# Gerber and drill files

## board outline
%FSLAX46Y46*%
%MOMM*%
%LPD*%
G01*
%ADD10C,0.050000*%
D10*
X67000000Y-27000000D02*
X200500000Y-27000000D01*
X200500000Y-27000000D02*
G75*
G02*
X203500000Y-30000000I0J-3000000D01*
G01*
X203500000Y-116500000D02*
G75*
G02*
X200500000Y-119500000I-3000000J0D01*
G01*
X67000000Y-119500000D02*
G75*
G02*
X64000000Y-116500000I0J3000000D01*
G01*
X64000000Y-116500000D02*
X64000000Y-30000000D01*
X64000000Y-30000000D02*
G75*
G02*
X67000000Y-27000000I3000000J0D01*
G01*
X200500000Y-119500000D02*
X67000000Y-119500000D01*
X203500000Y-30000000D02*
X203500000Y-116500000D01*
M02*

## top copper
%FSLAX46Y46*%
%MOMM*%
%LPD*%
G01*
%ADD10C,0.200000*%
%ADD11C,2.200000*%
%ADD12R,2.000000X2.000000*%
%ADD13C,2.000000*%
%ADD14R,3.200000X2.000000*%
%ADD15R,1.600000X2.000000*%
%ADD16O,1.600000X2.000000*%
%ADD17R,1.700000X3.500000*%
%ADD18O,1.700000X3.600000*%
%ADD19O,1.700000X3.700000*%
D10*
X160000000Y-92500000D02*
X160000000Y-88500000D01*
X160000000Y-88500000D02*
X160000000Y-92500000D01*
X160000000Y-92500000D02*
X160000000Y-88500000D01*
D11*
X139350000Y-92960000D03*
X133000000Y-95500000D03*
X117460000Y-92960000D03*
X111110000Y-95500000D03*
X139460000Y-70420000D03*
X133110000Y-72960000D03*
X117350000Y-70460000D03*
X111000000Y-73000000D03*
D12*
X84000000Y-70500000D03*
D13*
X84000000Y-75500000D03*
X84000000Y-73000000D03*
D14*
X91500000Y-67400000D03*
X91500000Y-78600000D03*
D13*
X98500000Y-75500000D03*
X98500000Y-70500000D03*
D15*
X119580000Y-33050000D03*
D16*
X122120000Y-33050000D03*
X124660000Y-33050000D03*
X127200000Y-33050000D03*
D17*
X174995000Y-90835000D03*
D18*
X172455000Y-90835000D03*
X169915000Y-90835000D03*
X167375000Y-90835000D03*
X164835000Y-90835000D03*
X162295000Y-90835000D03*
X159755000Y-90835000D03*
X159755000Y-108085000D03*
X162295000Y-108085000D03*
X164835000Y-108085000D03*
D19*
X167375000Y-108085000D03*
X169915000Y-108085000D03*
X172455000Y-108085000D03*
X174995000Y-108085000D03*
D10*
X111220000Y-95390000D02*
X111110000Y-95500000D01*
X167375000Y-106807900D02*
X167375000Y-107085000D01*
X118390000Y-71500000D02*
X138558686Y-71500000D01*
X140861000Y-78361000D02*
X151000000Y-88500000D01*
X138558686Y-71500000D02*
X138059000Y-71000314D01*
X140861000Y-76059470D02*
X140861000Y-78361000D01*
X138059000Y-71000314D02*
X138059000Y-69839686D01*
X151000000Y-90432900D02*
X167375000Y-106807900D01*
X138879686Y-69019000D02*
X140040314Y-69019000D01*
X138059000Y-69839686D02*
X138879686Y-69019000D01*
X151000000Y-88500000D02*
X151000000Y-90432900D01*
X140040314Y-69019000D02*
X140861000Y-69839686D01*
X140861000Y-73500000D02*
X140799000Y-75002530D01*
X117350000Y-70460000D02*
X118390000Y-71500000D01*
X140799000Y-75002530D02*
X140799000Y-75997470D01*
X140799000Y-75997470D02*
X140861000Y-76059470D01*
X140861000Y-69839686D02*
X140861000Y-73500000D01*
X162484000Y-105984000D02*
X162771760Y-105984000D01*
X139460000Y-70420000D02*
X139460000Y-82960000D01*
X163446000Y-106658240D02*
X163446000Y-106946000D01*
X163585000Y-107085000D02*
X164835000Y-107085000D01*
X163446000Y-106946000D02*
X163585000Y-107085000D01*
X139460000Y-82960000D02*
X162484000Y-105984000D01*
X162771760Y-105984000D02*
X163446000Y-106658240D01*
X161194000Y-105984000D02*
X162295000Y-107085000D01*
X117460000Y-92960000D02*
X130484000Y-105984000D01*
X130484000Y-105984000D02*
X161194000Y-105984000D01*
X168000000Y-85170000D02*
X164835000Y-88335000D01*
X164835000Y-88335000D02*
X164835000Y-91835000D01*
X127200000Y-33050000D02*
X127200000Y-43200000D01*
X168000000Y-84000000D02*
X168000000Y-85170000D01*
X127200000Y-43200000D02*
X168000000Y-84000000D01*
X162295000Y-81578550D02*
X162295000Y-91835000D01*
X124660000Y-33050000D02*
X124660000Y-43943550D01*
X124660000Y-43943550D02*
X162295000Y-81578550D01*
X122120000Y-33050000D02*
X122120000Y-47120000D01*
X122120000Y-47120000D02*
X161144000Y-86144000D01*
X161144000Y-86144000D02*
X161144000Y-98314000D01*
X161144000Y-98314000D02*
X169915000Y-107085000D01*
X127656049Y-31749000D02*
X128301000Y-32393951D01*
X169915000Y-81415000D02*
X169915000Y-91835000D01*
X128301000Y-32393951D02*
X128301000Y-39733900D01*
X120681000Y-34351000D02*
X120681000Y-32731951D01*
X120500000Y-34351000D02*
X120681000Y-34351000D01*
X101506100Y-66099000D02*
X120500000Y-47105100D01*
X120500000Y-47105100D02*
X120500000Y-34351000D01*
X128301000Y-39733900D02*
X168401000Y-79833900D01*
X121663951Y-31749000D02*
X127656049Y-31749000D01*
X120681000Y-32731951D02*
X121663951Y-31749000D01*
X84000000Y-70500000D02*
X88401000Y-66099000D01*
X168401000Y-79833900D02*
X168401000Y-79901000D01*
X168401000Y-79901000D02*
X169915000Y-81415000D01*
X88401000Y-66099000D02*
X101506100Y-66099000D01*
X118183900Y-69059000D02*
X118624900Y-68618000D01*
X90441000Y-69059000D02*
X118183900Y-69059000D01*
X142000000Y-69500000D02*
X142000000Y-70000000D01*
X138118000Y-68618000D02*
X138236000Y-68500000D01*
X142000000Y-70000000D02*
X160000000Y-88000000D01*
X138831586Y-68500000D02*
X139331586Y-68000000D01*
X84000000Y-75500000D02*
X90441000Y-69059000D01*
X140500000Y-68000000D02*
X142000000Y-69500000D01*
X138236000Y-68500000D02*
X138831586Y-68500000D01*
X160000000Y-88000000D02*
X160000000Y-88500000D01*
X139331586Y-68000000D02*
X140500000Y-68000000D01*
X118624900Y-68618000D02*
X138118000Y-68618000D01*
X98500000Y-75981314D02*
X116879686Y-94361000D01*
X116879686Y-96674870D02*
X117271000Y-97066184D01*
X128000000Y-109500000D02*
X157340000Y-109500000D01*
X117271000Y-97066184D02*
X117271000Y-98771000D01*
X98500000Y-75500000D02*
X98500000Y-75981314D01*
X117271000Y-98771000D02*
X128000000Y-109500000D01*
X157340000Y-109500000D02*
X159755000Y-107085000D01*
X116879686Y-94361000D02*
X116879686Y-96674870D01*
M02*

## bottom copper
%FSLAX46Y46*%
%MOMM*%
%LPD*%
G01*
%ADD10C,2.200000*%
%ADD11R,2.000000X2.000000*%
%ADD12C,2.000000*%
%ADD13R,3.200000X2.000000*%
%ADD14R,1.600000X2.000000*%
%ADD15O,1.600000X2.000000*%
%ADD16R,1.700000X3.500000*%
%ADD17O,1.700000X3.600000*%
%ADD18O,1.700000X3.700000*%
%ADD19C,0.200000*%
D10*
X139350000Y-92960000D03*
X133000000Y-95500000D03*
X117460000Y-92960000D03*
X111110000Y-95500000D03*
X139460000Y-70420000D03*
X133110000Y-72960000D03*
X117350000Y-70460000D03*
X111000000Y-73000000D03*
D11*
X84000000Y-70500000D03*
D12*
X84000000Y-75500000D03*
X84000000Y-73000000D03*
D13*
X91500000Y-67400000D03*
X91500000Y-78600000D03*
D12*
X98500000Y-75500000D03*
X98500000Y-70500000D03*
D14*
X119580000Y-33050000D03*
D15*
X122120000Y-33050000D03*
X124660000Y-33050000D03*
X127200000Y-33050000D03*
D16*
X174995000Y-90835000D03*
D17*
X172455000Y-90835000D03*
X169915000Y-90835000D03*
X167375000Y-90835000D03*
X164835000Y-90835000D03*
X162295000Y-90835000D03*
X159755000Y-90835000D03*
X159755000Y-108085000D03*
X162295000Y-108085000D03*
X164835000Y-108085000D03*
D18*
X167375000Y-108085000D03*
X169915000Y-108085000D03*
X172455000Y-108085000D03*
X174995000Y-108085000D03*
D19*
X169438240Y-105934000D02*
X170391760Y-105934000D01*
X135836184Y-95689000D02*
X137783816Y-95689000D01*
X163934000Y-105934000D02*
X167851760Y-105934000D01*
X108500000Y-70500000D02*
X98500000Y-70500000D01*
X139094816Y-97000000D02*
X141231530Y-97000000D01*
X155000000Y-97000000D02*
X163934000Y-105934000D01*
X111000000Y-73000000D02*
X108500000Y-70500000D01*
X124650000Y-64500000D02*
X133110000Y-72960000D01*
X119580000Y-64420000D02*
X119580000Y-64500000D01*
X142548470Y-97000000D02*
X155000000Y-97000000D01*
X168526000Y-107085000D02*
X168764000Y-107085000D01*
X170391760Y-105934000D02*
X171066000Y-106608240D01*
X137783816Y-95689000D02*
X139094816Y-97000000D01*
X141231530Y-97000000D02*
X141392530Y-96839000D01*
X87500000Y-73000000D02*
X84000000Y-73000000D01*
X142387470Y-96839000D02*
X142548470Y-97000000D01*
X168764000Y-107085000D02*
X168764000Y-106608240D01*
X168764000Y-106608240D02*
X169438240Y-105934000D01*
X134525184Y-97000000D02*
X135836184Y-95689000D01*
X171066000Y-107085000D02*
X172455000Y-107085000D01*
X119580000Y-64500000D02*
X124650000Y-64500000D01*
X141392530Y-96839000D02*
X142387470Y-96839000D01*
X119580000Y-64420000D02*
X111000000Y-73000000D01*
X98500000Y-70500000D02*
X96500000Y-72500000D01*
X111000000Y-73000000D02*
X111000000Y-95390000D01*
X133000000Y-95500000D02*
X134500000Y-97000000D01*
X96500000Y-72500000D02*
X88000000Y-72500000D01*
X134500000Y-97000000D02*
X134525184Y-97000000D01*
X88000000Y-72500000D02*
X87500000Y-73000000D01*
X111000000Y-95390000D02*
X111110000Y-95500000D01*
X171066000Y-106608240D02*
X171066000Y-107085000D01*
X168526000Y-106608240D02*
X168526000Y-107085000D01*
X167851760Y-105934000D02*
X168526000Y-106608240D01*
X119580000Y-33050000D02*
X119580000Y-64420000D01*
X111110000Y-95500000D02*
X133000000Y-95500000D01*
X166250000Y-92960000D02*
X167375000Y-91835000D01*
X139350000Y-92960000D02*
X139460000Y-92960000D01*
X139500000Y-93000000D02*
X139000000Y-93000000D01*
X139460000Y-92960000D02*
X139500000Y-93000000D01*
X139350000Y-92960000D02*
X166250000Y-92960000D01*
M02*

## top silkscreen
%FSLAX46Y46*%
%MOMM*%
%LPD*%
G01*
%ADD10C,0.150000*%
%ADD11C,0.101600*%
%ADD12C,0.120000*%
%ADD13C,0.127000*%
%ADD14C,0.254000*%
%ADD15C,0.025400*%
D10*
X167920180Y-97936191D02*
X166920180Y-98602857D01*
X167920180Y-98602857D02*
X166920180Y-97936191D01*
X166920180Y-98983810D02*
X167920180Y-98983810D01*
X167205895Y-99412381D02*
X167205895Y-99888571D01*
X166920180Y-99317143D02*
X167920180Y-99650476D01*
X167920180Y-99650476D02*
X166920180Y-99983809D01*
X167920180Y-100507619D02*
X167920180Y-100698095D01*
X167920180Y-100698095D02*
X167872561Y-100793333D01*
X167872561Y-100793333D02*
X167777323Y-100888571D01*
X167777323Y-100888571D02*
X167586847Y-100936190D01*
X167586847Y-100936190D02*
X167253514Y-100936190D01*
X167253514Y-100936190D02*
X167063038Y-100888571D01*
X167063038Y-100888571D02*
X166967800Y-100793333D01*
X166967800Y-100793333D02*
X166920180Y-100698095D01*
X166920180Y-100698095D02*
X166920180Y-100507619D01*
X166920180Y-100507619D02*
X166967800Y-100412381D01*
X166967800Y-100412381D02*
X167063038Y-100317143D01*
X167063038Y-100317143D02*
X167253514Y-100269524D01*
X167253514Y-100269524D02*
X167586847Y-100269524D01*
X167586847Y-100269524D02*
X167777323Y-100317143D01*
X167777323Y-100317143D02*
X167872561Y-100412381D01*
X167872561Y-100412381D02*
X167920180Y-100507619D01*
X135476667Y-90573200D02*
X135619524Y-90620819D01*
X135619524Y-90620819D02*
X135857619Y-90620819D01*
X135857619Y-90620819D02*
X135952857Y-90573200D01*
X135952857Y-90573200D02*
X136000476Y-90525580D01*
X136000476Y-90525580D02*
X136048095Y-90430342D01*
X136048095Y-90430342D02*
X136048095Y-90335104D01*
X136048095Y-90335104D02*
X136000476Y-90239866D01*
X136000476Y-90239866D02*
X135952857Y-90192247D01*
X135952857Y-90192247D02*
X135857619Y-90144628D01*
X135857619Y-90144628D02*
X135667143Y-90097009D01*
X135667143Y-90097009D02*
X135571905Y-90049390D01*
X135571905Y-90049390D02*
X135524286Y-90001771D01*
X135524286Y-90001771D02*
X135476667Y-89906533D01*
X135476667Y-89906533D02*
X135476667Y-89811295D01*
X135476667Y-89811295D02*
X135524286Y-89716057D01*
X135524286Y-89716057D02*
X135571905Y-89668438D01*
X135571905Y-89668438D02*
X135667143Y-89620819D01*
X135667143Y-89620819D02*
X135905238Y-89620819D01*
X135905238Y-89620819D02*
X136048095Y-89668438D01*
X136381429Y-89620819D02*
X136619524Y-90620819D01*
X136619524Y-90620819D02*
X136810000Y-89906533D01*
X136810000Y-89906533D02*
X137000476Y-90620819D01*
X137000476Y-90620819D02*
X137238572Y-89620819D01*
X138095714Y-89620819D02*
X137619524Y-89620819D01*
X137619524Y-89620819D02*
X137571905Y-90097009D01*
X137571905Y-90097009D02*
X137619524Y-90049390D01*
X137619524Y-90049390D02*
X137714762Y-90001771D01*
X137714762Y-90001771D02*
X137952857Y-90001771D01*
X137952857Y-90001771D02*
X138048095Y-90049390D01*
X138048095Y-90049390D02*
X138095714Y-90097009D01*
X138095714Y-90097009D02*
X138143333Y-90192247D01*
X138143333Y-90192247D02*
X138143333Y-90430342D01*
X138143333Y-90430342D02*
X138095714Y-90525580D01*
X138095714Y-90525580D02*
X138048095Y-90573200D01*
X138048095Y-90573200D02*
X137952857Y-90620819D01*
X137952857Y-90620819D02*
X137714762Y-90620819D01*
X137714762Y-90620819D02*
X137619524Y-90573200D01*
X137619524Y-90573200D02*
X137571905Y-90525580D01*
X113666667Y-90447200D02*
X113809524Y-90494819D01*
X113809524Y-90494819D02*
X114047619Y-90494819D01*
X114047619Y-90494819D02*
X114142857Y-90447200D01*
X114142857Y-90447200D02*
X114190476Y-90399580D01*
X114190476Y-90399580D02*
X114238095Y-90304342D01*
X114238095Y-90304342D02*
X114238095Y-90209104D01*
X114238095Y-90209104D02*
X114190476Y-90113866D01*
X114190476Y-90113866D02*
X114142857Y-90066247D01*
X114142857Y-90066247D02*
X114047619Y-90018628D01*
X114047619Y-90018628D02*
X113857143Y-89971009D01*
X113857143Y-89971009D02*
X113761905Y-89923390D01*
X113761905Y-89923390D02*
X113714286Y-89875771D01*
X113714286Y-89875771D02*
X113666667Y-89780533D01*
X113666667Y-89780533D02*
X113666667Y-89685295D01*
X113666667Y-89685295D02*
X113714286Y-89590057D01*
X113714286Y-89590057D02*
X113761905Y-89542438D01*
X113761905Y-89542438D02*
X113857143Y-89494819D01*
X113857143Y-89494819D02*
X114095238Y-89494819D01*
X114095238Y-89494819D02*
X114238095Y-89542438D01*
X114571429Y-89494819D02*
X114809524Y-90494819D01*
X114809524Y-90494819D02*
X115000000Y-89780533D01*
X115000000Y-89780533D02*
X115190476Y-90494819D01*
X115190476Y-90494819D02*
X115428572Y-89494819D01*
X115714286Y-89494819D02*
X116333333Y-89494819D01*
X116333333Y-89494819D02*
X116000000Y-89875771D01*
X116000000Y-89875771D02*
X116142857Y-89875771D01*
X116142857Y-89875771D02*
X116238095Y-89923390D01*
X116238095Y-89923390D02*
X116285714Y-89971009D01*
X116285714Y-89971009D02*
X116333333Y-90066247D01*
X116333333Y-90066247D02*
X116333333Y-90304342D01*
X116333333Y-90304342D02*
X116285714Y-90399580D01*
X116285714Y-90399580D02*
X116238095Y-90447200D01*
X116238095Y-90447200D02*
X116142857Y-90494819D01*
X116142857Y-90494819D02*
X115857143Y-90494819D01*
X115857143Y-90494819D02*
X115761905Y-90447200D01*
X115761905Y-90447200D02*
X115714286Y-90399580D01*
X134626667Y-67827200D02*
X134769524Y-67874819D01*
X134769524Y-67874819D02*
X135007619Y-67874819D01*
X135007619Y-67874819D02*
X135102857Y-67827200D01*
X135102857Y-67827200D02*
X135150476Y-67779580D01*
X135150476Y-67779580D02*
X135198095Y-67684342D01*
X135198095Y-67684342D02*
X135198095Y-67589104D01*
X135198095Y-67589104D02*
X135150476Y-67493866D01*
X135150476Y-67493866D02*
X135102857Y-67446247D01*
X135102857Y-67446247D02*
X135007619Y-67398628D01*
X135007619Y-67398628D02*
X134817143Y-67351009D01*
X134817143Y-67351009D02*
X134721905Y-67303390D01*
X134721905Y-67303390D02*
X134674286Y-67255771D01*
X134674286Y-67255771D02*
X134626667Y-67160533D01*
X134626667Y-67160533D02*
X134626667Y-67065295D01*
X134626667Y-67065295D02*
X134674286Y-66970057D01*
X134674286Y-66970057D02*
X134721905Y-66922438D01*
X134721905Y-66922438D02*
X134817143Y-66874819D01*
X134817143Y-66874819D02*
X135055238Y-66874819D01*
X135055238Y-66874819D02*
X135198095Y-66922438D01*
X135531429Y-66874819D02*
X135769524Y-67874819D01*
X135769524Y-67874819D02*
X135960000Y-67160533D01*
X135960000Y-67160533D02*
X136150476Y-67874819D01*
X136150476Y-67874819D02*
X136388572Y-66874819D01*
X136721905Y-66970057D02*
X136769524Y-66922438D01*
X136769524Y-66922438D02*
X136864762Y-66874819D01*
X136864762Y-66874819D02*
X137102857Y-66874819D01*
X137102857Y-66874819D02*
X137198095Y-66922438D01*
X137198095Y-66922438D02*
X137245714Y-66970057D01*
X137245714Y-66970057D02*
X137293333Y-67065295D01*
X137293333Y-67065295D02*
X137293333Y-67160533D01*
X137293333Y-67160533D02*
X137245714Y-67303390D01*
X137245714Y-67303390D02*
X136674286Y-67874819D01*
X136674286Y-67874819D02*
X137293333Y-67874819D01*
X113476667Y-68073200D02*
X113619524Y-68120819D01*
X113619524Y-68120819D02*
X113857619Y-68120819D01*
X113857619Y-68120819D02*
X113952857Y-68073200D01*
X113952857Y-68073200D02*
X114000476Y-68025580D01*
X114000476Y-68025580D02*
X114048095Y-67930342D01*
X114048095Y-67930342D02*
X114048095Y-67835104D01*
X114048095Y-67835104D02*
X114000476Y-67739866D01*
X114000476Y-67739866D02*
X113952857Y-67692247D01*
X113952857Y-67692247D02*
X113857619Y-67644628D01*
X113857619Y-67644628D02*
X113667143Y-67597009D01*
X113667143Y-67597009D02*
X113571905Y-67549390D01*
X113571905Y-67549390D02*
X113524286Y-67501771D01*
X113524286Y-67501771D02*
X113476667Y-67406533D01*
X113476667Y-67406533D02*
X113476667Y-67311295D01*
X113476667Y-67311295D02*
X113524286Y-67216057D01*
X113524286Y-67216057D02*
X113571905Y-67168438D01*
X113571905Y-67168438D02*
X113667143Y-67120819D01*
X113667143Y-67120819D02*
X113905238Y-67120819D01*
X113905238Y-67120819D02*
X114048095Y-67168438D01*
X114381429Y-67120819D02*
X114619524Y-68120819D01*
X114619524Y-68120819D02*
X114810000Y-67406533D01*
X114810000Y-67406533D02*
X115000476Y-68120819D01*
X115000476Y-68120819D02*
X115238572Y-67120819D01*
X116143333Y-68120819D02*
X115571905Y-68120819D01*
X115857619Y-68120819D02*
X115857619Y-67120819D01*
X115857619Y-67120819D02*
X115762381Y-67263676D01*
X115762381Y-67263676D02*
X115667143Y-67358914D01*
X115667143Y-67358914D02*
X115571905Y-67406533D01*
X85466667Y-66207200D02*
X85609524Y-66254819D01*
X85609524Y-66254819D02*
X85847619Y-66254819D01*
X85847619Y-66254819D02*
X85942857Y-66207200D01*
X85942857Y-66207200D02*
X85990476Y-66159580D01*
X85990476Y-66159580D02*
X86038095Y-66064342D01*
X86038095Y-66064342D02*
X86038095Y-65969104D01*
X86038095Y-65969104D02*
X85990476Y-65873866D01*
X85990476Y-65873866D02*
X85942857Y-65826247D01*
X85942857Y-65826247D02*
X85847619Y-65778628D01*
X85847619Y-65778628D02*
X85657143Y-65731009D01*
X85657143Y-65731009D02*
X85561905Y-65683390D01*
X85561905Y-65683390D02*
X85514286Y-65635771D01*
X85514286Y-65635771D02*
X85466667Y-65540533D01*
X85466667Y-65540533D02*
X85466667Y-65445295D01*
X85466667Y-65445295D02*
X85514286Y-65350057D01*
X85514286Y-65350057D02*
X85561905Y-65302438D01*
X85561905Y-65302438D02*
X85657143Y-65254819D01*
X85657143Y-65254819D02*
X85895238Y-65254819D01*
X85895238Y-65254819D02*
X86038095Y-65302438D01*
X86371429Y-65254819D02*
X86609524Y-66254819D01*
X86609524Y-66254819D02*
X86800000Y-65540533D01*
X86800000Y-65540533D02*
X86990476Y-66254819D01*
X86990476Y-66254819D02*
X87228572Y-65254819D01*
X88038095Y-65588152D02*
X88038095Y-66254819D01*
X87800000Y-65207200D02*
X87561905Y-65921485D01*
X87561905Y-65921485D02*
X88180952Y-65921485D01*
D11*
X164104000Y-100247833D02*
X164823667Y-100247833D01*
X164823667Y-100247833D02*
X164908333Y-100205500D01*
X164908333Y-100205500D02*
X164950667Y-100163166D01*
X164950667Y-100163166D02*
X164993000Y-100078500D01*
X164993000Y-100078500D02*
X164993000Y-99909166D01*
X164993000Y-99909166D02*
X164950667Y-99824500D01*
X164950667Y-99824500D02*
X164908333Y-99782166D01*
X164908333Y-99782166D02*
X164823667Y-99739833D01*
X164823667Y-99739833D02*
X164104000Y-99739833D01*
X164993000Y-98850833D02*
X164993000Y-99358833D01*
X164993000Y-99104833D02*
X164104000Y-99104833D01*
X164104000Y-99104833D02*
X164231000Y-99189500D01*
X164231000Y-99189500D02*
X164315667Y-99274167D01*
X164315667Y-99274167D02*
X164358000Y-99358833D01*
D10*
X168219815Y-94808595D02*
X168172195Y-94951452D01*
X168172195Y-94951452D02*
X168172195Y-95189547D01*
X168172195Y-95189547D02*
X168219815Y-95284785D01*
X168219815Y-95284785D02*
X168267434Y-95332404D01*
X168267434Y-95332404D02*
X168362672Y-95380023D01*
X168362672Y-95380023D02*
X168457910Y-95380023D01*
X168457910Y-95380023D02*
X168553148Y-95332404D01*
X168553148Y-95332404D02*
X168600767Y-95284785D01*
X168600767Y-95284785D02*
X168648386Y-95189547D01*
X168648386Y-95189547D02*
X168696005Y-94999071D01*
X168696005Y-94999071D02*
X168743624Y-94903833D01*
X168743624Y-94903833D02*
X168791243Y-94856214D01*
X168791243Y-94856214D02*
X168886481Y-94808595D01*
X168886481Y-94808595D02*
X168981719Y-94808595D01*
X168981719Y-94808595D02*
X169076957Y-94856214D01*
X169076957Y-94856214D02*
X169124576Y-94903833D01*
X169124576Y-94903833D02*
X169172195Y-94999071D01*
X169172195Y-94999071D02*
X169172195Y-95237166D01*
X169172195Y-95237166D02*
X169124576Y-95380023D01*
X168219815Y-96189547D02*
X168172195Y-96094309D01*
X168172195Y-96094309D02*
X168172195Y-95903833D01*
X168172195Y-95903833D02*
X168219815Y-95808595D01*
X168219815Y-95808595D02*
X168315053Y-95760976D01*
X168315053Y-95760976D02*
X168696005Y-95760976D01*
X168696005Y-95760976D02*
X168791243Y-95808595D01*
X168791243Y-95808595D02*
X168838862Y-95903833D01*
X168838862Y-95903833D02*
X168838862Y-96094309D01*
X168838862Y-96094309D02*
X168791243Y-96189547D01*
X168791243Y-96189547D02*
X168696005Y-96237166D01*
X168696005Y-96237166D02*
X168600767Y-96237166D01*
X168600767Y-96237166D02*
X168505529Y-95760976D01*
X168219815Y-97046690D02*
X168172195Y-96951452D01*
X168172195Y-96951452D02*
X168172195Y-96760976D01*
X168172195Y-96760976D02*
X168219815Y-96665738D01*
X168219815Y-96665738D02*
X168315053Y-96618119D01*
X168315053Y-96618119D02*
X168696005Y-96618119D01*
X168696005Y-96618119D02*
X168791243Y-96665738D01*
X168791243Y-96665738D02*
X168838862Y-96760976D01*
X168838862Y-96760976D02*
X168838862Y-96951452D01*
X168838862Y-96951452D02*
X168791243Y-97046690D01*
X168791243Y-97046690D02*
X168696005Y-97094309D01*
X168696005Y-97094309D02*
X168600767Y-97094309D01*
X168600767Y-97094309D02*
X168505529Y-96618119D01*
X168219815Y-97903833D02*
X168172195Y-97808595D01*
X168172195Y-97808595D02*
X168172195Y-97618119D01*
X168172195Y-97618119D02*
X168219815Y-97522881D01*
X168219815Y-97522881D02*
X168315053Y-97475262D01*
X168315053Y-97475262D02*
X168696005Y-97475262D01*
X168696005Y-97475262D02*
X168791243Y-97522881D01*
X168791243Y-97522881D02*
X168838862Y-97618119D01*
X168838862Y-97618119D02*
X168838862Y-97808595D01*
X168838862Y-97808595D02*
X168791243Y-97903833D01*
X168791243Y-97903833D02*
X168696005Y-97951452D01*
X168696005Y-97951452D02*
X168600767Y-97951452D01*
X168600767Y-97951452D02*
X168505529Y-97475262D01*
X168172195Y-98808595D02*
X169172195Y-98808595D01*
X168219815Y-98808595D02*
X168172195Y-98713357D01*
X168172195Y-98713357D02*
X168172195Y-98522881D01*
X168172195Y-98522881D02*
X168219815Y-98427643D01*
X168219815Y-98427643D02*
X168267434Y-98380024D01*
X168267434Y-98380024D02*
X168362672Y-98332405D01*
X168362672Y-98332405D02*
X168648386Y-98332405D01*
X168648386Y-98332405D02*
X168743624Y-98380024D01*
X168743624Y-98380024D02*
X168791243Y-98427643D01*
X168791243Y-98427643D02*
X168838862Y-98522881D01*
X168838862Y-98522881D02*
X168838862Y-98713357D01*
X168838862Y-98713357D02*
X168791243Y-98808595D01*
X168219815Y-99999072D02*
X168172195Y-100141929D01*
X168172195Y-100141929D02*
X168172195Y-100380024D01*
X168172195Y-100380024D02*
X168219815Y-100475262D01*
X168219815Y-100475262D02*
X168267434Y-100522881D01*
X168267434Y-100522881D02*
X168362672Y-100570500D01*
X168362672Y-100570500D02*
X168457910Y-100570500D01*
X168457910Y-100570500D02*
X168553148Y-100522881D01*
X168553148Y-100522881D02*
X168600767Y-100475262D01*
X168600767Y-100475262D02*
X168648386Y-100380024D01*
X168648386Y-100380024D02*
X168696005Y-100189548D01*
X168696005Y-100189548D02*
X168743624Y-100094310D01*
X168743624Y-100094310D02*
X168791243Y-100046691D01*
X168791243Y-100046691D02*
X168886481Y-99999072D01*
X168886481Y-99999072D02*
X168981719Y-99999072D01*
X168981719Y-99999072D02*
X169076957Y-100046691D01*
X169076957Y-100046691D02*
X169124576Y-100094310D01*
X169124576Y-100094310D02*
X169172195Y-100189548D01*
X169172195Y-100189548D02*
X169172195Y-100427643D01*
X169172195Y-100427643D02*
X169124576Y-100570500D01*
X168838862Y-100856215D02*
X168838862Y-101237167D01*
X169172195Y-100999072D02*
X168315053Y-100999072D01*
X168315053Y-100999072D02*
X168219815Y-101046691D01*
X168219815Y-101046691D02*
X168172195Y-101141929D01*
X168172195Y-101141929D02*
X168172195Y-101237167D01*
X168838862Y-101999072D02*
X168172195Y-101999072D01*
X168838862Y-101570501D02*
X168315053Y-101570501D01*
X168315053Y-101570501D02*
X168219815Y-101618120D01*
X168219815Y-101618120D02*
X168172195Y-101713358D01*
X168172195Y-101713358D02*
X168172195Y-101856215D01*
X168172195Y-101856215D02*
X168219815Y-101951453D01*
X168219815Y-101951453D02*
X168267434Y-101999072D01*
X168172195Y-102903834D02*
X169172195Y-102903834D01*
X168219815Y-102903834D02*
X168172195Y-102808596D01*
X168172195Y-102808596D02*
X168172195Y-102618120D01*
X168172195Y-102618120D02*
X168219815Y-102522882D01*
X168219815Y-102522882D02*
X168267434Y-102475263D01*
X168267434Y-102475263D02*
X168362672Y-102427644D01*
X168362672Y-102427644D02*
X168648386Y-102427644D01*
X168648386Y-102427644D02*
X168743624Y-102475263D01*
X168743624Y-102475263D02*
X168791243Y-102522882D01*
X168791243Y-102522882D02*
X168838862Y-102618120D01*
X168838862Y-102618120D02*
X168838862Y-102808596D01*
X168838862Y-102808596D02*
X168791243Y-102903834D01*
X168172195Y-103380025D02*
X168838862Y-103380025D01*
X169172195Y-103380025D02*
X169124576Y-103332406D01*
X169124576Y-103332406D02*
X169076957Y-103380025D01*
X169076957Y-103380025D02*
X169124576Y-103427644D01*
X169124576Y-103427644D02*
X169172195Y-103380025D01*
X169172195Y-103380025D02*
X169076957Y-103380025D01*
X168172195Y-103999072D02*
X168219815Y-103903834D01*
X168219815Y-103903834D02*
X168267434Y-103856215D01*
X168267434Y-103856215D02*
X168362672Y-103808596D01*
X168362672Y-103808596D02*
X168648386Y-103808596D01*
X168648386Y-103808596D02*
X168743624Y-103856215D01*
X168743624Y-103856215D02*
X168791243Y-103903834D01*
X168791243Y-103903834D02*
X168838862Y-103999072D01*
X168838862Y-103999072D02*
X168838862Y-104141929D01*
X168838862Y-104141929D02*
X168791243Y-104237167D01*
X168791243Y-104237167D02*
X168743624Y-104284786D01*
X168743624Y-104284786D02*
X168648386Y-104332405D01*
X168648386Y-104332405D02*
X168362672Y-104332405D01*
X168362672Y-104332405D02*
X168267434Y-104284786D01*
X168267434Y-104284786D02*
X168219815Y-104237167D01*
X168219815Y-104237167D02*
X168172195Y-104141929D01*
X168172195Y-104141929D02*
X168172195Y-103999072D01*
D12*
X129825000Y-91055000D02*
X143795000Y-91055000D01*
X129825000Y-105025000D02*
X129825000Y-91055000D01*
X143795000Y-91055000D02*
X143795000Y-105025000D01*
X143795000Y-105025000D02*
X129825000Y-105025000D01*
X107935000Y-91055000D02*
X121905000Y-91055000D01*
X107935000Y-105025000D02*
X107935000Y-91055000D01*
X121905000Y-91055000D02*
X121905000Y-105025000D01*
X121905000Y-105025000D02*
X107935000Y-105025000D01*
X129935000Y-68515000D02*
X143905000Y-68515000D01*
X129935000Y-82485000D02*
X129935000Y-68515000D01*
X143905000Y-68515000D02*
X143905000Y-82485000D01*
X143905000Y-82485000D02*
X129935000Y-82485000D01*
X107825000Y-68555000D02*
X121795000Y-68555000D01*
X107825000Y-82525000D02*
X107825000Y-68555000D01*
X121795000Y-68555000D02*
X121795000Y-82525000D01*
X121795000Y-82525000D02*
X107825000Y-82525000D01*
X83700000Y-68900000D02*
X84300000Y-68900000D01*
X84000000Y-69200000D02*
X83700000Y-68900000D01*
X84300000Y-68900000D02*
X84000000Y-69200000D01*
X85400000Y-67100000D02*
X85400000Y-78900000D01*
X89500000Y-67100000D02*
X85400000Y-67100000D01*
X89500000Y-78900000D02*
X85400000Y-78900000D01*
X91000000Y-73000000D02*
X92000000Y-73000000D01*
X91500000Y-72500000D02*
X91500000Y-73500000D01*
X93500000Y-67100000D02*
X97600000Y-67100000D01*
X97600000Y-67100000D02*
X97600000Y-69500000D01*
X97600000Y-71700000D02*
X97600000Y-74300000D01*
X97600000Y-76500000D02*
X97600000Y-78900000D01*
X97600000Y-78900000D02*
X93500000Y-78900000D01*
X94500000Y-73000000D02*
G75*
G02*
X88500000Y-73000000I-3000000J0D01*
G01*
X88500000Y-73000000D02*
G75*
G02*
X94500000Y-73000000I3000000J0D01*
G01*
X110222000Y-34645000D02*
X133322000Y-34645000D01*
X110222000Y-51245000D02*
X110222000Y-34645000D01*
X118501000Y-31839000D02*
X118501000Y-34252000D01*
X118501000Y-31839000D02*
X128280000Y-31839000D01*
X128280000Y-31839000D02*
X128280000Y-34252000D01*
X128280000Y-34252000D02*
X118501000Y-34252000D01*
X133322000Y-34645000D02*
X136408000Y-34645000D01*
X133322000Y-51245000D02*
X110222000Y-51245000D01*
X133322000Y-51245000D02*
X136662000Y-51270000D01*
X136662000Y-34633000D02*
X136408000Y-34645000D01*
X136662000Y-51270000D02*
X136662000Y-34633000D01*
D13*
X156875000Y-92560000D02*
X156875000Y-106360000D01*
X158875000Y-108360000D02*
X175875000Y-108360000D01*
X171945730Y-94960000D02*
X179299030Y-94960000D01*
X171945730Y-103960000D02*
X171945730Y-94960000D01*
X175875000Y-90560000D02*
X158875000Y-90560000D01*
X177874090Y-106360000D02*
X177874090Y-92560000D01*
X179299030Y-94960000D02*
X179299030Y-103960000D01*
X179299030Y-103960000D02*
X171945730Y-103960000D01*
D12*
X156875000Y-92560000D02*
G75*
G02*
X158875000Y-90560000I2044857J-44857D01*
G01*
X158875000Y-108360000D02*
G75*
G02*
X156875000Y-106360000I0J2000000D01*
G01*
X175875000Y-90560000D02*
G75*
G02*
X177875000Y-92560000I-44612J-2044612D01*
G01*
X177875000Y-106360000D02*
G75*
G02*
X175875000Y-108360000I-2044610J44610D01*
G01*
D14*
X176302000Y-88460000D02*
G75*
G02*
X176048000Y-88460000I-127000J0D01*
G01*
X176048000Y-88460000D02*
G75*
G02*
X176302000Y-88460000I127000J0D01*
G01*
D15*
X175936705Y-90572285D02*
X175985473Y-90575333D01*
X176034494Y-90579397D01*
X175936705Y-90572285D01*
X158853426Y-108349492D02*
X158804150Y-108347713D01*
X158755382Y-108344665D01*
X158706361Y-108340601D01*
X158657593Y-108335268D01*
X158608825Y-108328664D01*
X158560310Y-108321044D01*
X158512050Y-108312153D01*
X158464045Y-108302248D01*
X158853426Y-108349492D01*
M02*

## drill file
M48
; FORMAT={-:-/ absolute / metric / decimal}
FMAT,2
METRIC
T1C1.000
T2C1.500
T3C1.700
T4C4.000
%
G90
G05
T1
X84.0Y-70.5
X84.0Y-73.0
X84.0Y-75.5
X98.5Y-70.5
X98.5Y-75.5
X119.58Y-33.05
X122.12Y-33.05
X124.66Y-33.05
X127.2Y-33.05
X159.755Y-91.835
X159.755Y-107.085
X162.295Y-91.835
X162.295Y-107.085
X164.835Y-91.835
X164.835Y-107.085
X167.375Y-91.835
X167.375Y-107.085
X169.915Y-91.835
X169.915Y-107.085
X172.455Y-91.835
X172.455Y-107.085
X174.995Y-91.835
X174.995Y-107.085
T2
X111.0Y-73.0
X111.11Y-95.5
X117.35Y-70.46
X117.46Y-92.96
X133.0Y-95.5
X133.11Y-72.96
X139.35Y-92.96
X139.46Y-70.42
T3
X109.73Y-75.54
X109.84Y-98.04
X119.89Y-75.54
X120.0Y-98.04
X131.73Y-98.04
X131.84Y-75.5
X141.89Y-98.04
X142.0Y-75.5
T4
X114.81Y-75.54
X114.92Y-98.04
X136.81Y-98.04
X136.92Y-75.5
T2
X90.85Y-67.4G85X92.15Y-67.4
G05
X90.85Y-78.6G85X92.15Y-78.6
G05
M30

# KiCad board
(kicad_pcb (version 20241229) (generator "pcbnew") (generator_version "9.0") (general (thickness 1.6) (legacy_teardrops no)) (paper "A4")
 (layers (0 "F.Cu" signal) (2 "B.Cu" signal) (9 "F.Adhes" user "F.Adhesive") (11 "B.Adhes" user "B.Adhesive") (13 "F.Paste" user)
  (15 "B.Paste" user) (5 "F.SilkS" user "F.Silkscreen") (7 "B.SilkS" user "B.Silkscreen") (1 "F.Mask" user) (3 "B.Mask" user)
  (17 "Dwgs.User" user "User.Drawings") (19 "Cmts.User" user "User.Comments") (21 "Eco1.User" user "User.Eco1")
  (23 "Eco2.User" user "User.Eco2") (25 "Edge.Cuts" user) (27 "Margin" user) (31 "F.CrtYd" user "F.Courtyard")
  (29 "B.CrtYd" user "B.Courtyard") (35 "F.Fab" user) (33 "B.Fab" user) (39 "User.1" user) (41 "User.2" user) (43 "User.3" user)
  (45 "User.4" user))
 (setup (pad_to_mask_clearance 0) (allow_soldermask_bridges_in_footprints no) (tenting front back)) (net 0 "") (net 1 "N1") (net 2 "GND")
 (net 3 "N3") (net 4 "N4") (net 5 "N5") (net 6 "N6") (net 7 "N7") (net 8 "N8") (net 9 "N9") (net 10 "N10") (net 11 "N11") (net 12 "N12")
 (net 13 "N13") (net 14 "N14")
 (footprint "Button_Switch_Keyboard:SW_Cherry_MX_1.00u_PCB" (layer "F.Cu") (at 139.35 92.96)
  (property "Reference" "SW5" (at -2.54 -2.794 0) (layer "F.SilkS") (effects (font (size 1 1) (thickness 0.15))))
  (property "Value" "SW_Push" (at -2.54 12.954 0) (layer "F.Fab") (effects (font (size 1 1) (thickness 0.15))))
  (fp_line (start -9.525 -1.905) (end 4.445 -1.905) (stroke (width 0.12) (type solid)) (layer "F.SilkS"))
  (fp_line (start -9.525 12.065) (end -9.525 -1.905) (stroke (width 0.12) (type solid)) (layer "F.SilkS"))
  (fp_line (start 4.445 -1.905) (end 4.445 12.065) (stroke (width 0.12) (type solid)) (layer "F.SilkS"))
  (fp_line (start 4.445 12.065) (end -9.525 12.065) (stroke (width 0.12) (type solid)) (layer "F.SilkS"))
  (pad "" np_thru_hole circle (at -7.62 5.08) (size 1.7 1.7) (drill 1.7) (layers "*.Cu" "*.Mask"))
  (pad "" np_thru_hole circle (at -2.54 5.08) (size 4 4) (drill 4) (layers "*.Cu" "*.Mask"))
  (pad "" np_thru_hole circle (at 2.54 5.08) (size 1.7 1.7) (drill 1.7) (layers "*.Cu" "*.Mask"))
  (pad "1" thru_hole circle (at 0 0) (size 2.2 2.2) (drill 1.5) (layers "*.Cu" "*.Mask") (remove_unused_layers no) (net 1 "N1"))
  (pad "2" thru_hole circle (at -6.35 2.54) (size 2.2 2.2) (drill 1.5) (layers "*.Cu" "*.Mask") (remove_unused_layers no) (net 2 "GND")))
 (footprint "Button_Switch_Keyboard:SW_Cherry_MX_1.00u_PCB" (layer "F.Cu") (at 117.46 92.96)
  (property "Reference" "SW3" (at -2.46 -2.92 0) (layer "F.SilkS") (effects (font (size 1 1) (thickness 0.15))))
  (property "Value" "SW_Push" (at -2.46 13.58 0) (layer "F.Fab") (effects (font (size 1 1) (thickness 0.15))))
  (fp_line (start -9.525 -1.905) (end 4.445 -1.905) (stroke (width 0.12) (type solid)) (layer "F.SilkS"))
  (fp_line (start -9.525 12.065) (end -9.525 -1.905) (stroke (width 0.12) (type solid)) (layer "F.SilkS"))
  (fp_line (start 4.445 -1.905) (end 4.445 12.065) (stroke (width 0.12) (type solid)) (layer "F.SilkS"))
  (fp_line (start 4.445 12.065) (end -9.525 12.065) (stroke (width 0.12) (type solid)) (layer "F.SilkS"))
  (pad "" np_thru_hole circle (at -7.62 5.08) (size 1.7 1.7) (drill 1.7) (layers "*.Cu" "*.Mask"))
  (pad "" np_thru_hole circle (at -2.54 5.08) (size 4 4) (drill 4) (layers "*.Cu" "*.Mask"))
  (pad "" np_thru_hole circle (at 2.54 5.08) (size 1.7 1.7) (drill 1.7) (layers "*.Cu" "*.Mask"))
  (pad "1" thru_hole circle (at 0 0) (size 2.2 2.2) (drill 1.5) (layers "*.Cu" "*.Mask") (remove_unused_layers no) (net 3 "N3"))
  (pad "2" thru_hole circle (at -6.35 2.54) (size 2.2 2.2) (drill 1.5) (layers "*.Cu" "*.Mask") (remove_unused_layers no) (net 2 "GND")))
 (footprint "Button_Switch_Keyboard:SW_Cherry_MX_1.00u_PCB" (layer "F.Cu") (at 139.46 70.42)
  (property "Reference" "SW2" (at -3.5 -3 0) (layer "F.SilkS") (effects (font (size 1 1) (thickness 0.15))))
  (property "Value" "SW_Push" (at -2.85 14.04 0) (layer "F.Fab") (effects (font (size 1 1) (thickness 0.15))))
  (fp_line (start -9.525 -1.905) (end 4.445 -1.905) (stroke (width 0.12) (type solid)) (layer "F.SilkS"))
  (fp_line (start -9.525 12.065) (end -9.525 -1.905) (stroke (width 0.12) (type solid)) (layer "F.SilkS"))
  (fp_line (start 4.445 -1.905) (end 4.445 12.065) (stroke (width 0.12) (type solid)) (layer "F.SilkS"))
  (fp_line (start 4.445 12.065) (end -9.525 12.065) (stroke (width 0.12) (type solid)) (layer "F.SilkS"))
  (pad "" np_thru_hole circle (at -7.62 5.08) (size 1.7 1.7) (drill 1.7) (layers "*.Cu" "*.Mask"))
  (pad "" np_thru_hole circle (at -2.54 5.08) (size 4 4) (drill 4) (layers "*.Cu" "*.Mask"))
  (pad "" np_thru_hole circle (at 2.54 5.08) (size 1.7 1.7) (drill 1.7) (layers "*.Cu" "*.Mask"))
  (pad "1" thru_hole circle (at 0 0) (size 2.2 2.2) (drill 1.5) (layers "*.Cu" "*.Mask") (remove_unused_layers no) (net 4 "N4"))
  (pad "2" thru_hole circle (at -6.35 2.54) (size 2.2 2.2) (drill 1.5) (layers "*.Cu" "*.Mask") (remove_unused_layers no) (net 2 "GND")))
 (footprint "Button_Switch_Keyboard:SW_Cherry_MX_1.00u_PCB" (layer "F.Cu") (at 117.35 70.46)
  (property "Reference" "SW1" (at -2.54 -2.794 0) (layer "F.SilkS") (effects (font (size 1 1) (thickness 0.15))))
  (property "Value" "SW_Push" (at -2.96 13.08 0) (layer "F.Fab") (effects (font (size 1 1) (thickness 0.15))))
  (fp_line (start -9.525 -1.905) (end 4.445 -1.905) (stroke (width 0.12) (type solid)) (layer "F.SilkS"))
  (fp_line (start -9.525 12.065) (end -9.525 -1.905) (stroke (width 0.12) (type solid)) (layer "F.SilkS"))
  (fp_line (start 4.445 -1.905) (end 4.445 12.065) (stroke (width 0.12) (type solid)) (layer "F.SilkS"))
  (fp_line (start 4.445 12.065) (end -9.525 12.065) (stroke (width 0.12) (type solid)) (layer "F.SilkS"))
  (pad "" np_thru_hole circle (at -7.62 5.08) (size 1.7 1.7) (drill 1.7) (layers "*.Cu" "*.Mask"))
  (pad "" np_thru_hole circle (at -2.54 5.08) (size 4 4) (drill 4) (layers "*.Cu" "*.Mask"))
  (pad "" np_thru_hole circle (at 2.54 5.08) (size 1.7 1.7) (drill 1.7) (layers "*.Cu" "*.Mask"))
  (pad "1" thru_hole circle (at 0 0) (size 2.2 2.2) (drill 1.5) (layers "*.Cu" "*.Mask") (remove_unused_layers no) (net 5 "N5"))
  (pad "2" thru_hole circle (at -6.35 2.54) (size 2.2 2.2) (drill 1.5) (layers "*.Cu" "*.Mask") (remove_unused_layers no) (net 2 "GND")))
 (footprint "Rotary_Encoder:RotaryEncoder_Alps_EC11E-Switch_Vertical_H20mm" (layer "F.Cu") (at 84 70.5)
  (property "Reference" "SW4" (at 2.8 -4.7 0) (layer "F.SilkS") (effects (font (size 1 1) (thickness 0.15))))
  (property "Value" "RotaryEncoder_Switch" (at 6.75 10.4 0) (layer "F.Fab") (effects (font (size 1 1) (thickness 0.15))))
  (fp_line (start -0.3 -1.6) (end 0.3 -1.6) (stroke (width 0.12) (type solid)) (layer "F.SilkS"))
  (fp_line (start 0 -1.3) (end -0.3 -1.6) (stroke (width 0.12) (type solid)) (layer "F.SilkS"))
  (fp_line (start 0.3 -1.6) (end 0 -1.3) (stroke (width 0.12) (type solid)) (layer "F.SilkS"))
  (fp_line (start 1.4 -3.4) (end 1.4 8.4) (stroke (width 0.12) (type solid)) (layer "F.SilkS"))
  (fp_line (start 5.5 -3.4) (end 1.4 -3.4) (stroke (width 0.12) (type solid)) (layer "F.SilkS"))
  (fp_line (start 5.5 8.4) (end 1.4 8.4) (stroke (width 0.12) (type solid)) (layer "F.SilkS"))
  (fp_line (start 7 2.5) (end 8 2.5) (stroke (width 0.12) (type solid)) (layer "F.SilkS"))
  (fp_line (start 7.5 2) (end 7.5 3) (stroke (width 0.12) (type solid)) (layer "F.SilkS"))
  (fp_line (start 9.5 -3.4) (end 13.6 -3.4) (stroke (width 0.12) (type solid)) (layer "F.SilkS"))
  (fp_line (start 13.6 -3.4) (end 13.6 -1) (stroke (width 0.12) (type solid)) (layer "F.SilkS"))
  (fp_line (start 13.6 1.2) (end 13.6 3.8) (stroke (width 0.12) (type solid)) (layer "F.SilkS"))
  (fp_line (start 13.6 6) (end 13.6 8.4) (stroke (width 0.12) (type solid)) (layer "F.SilkS"))
  (fp_line (start 13.6 8.4) (end 9.5 8.4) (stroke (width 0.12) (type solid)) (layer "F.SilkS"))
  (fp_circle (center 7.5 2.5) (end 10.5 2.5) (stroke (width 0.12) (type solid)) (fill no) (layer "F.SilkS"))
  (pad "A" thru_hole rect (at 0 0) (size 2 2) (drill 1) (layers "*.Cu" "*.Mask") (remove_unused_layers no) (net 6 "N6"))
  (pad "B" thru_hole circle (at 0 5) (size 2 2) (drill 1) (layers "*.Cu" "*.Mask") (remove_unused_layers no) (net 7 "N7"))
  (pad "C" thru_hole circle (at 0 2.5) (size 2 2) (drill 1) (layers "*.Cu" "*.Mask") (remove_unused_layers no) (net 2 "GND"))
  (pad "MP" thru_hole rect (at 7.5 -3.1) (size 3.2 2) (drill oval 2.8 1.5) (layers "*.Cu" "*.Mask") (remove_unused_layers no))
  (pad "MP" thru_hole rect (at 7.5 8.1) (size 3.2 2) (drill oval 2.8 1.5) (layers "*.Cu" "*.Mask") (remove_unused_layers no))
  (pad "S1" thru_hole circle (at 14.5 5) (size 2 2) (drill 1) (layers "*.Cu" "*.Mask") (remove_unused_layers no) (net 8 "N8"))
  (pad "S2" thru_hole circle (at 14.5 0) (size 2 2) (drill 1) (layers "*.Cu" "*.Mask") (remove_unused_layers no) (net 2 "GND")))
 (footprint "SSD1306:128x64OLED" (layer "F.Cu") (at 123.2 43.65)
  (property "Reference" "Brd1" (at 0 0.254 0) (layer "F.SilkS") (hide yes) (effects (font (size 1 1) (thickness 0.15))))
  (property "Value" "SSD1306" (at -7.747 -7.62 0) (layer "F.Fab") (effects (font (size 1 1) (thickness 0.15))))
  (fp_line (start -12.978 -9.005) (end 10.122 -9.005) (stroke (width 0.12) (type solid)) (layer "F.SilkS"))
  (fp_line (start -12.978 7.595) (end -12.978 -9.005) (stroke (width 0.12) (type solid)) (layer "F.SilkS"))
  (fp_line (start -4.699 -11.811) (end -4.699 -9.398) (stroke (width 0.12) (type solid)) (layer "F.SilkS"))
  (fp_line (start -4.699 -11.811) (end 5.08 -11.811) (stroke (width 0.12) (type solid)) (layer "F.SilkS"))
  (fp_line (start 5.08 -11.811) (end 5.08 -9.398) (stroke (width 0.12) (type solid)) (layer "F.SilkS"))
  (fp_line (start 5.08 -9.398) (end -4.699 -9.398) (stroke (width 0.12) (type solid)) (layer "F.SilkS"))
  (fp_line (start 10.122 -9.005) (end 13.208 -9.005) (stroke (width 0.12) (type solid)) (layer "F.SilkS"))
  (fp_line (start 10.122 7.595) (end -12.978 7.595) (stroke (width 0.12) (type solid)) (layer "F.SilkS"))
  (fp_line (start 10.122 7.595) (end 13.462 7.62) (stroke (width 0.12) (type solid)) (layer "F.SilkS"))
  (fp_line (start 13.462 -9.017) (end 13.208 -9.005) (stroke (width 0.12) (type solid)) (layer "F.SilkS"))
  (fp_line (start 13.462 7.62) (end 13.462 -9.017) (stroke (width 0.12) (type solid)) (layer "F.SilkS"))
  (pad "1" thru_hole rect (at -3.62 -10.6 90) (size 2 1.6) (drill 1) (layers "*.Cu" "*.Mask") (remove_unused_layers no) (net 2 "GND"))
  (pad "2" thru_hole oval (at -1.08 -10.6 90) (size 2 1.6) (drill 1) (layers "*.Cu" "*.Mask") (remove_unused_layers no) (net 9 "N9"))
  (pad "3" thru_hole oval (at 1.46 -10.6 90) (size 2 1.6) (drill 1) (layers "*.Cu" "*.Mask") (remove_unused_layers no) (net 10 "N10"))
  (pad "4" thru_hole oval (at 4 -10.6 90) (size 2 1.6) (drill 1) (layers "*.Cu" "*.Mask") (remove_unused_layers no) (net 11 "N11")))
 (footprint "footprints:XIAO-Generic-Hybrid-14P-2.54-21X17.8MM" (layer "F.Cu") (at 167.375 99.46 -90)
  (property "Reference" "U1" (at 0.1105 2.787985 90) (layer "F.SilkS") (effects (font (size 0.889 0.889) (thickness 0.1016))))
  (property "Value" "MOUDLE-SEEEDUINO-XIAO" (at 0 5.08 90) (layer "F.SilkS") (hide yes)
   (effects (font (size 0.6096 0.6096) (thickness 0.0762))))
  (fp_line (start -6.9 10.5) (end 6.9 10.5) (stroke (width 0.127) (type solid)) (layer "F.SilkS"))
  (fp_line (start 8.9 8.5) (end 8.9 -8.5) (stroke (width 0.127) (type solid)) (layer "F.SilkS"))
  (fp_line (start -4.5 -4.57073) (end -4.5 -11.92403) (stroke (width 0.127) (type solid)) (layer "F.SilkS"))
  (fp_line (start 4.5 -4.57073) (end -4.5 -4.57073) (stroke (width 0.127) (type solid)) (layer "F.SilkS"))
  (fp_line (start -8.9 -8.5) (end -8.9 8.5) (stroke (width 0.127) (type solid)) (layer "F.SilkS"))
  (fp_line (start 6.9 -10.49909) (end -6.9 -10.49909) (stroke (width 0.127) (type solid)) (layer "F.SilkS"))
  (fp_line (start -4.5 -11.92403) (end 4.5 -11.92403) (stroke (width 0.127) (type solid)) (layer "F.SilkS"))
  (fp_line (start 4.5 -11.92403) (end 4.5 -4.57073) (stroke (width 0.127) (type solid)) (layer "F.SilkS"))
  (fp_arc (start -6.9 10.5) (mid -8.301423 9.901423) (end -8.9 8.5) (stroke (width 0.12) (type solid)) (layer "F.SilkS"))
  (fp_arc (start 8.9 8.5) (mid 8.314214 9.914214) (end 6.9 10.5) (stroke (width 0.12) (type solid)) (layer "F.SilkS"))
  (fp_arc (start -8.9 -8.5) (mid -8.301491 -9.901491) (end -6.9 -10.5) (stroke (width 0.12) (type solid)) (layer "F.SilkS"))
  (fp_arc (start 6.9 -10.5) (mid 8.301491 -9.901491) (end 8.9 -8.5) (stroke (width 0.12) (type solid)) (layer "F.SilkS"))
  (fp_circle (center -11 -8.8) (end -11 -9.054) (stroke (width 0) (type solid)) (fill yes) (layer "F.SilkS"))
  (fp_poly
   (pts (xy -8.887715 -8.561705) (xy -8.884667 -8.610473) (xy -8.880603 -8.659494)) (stroke (width 0.0254) (type solid)) (fill no)
   (layer "F.SilkS"))
  (fp_poly
   (pts (xy 8.889492 8.521574) (xy 8.887713 8.57085) (xy 8.884665 8.619618) (xy 8.880601 8.668639) (xy 8.875268 8.717407)
    (xy 8.868664 8.766175) (xy 8.861044 8.81469) (xy 8.852153 8.86295) (xy 8.842248 8.910955))
   (stroke (width 0.0254) (type solid)) (fill no) (layer "F.SilkS"))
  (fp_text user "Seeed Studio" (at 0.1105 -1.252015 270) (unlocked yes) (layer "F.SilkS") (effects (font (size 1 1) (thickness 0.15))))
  (pad "1" thru_hole rect (at -7.625 -7.62 270) (size 3.5 1.7) (drill 1 (offset -1 0)) (layers "*.Cu" "*.Mask") (remove_unused_layers no)
   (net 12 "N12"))
  (pad "2" thru_hole oval (at -7.625 -5.08 270) (size 3.6 1.7) (drill 1 (offset -1 0)) (layers "*.Cu" "*.Mask") (remove_unused_layers no)
   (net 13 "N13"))
  (pad "3" thru_hole oval (at -7.625 -2.54 270) (size 3.6 1.7) (drill 1 (offset -1 0)) (layers "*.Cu" "*.Mask") (remove_unused_layers no)
   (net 6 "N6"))
  (pad "4" thru_hole oval (at -7.625 0 270) (size 3.6 1.7) (drill 1 (offset -1 0)) (layers "*.Cu" "*.Mask") (remove_unused_layers no)
   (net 1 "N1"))
  (pad "5" thru_hole oval (at -7.625 2.54 270) (size 3.6 1.7) (drill 1 (offset -1 0)) (layers "*.Cu" "*.Mask") (remove_unused_layers no)
   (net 11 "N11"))
  (pad "6" thru_hole oval (at -7.625 5.08 90) (size 3.6 1.7) (drill 1 (offset 1 0)) (layers "*.Cu" "*.Mask") (remove_unused_layers no)
   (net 10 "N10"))
  (pad "7" thru_hole oval (at -7.625 7.62 270) (size 3.6 1.7) (drill 1 (offset -1 0)) (layers "*.Cu" "*.Mask") (remove_unused_layers no)
   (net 7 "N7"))
  (pad "8" thru_hole oval (at 7.625 7.62 270) (size 3.6 1.7) (drill 1 (offset 1 0)) (layers "*.Cu" "*.Mask") (remove_unused_layers no)
   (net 8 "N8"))
  (pad "9" thru_hole oval (at 7.625 5.08 270) (size 3.6 1.7) (drill 1 (offset 1 0)) (layers "*.Cu" "*.Mask") (remove_unused_layers no)
   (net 3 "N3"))
  (pad "10" thru_hole oval (at 7.625 2.54 270) (size 3.6 1.7) (drill 1 (offset 1 0)) (layers "*.Cu" "*.Mask") (remove_unused_layers no)
   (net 4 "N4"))
  (pad "11" thru_hole oval (at 7.625 0 270) (size 3.7 1.7) (drill 1 (offset 1 0)) (layers "*.Cu" "*.Mask") (remove_unused_layers no)
   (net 5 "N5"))
  (pad "12" thru_hole oval (at 7.625 -2.54 270) (size 3.7 1.7) (drill 1 (offset 1 0)) (layers "*.Cu" "*.Mask") (remove_unused_layers no)
   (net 9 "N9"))
  (pad "13" thru_hole oval (at 7.625 -5.08 270) (size 3.7 1.7) (drill 1 (offset 1 0)) (layers "*.Cu" "*.Mask") (remove_unused_layers no)
   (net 2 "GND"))
  (pad "14" thru_hole oval (at 7.625 -7.62 270) (size 3.7 1.7) (drill 1 (offset 1 0)) (layers "*.Cu" "*.Mask") (remove_unused_layers no)
   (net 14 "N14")))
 (gr_line (start 160 92.5) (end 160 88.5) (stroke (width 0.2) (type default)) (layer "F.Cu") (net 7))
 (gr_line (start 160 88.5) (end 160 92.5) (stroke (width 0.2) (type default)) (layer "F.Cu") (net 7))
 (gr_line (start 160 92.5) (end 160 88.5) (stroke (width 0.2) (type default)) (layer "F.Cu") (net 7))
 (gr_line (start 67 27) (end 200.5 27) (stroke (width 0.05) (type default)) (layer "Edge.Cuts"))
 (gr_arc (start 200.5 27) (mid 202.62132 27.87868) (end 203.5 30) (stroke (width 0.05) (type default)) (layer "Edge.Cuts"))
 (gr_arc (start 203.5 116.5) (mid 202.62132 118.62132) (end 200.5 119.5) (stroke (width 0.05) (type default)) (layer "Edge.Cuts"))
 (gr_arc (start 67 119.5) (mid 64.87868 118.62132) (end 64 116.5) (stroke (width 0.05) (type default)) (layer "Edge.Cuts"))
 (gr_line (start 64 116.5) (end 64 30) (stroke (width 0.05) (type default)) (layer "Edge.Cuts"))
 (gr_arc (start 64 30) (mid 64.87868 27.87868) (end 67 27) (stroke (width 0.05) (type default)) (layer "Edge.Cuts"))
 (gr_line (start 200.5 119.5) (end 67 119.5) (stroke (width 0.05) (type default)) (layer "Edge.Cuts"))
 (gr_line (start 203.5 30) (end 203.5 116.5) (stroke (width 0.05) (type default)) (layer "Edge.Cuts"))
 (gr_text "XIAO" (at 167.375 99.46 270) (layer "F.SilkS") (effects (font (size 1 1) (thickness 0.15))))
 (segment (start 111.22 95.39) (end 111.11 95.5) (width 0.2) (layer "F.Cu") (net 2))
 (segment (start 169.43824 105.934) (end 170.39176 105.934) (width 0.2) (layer "B.Cu") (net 2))
 (segment (start 135.836184 95.689) (end 137.783816 95.689) (width 0.2) (layer "B.Cu") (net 2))
 (segment (start 163.934 105.934) (end 167.85176 105.934) (width 0.2) (layer "B.Cu") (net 2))
 (segment (start 108.5 70.5) (end 98.5 70.5) (width 0.2) (layer "B.Cu") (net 2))
 (segment (start 139.094816 97) (end 141.23153 97) (width 0.2) (layer "B.Cu") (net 2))
 (segment (start 155 97) (end 163.934 105.934) (width 0.2) (layer "B.Cu") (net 2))
 (segment (start 111 73) (end 108.5 70.5) (width 0.2) (layer "B.Cu") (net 2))
 (segment (start 124.65 64.5) (end 133.11 72.96) (width 0.2) (layer "B.Cu") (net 2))
 (segment (start 119.58 64.42) (end 119.58 64.5) (width 0.2) (layer "B.Cu") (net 2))
 (segment (start 142.54847 97) (end 155 97) (width 0.2) (layer "B.Cu") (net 2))
 (segment (start 168.526 107.085) (end 168.764 107.085) (width 0.2) (layer "B.Cu") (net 2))
 (segment (start 170.39176 105.934) (end 171.066 106.60824) (width 0.2) (layer "B.Cu") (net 2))
 (segment (start 137.783816 95.689) (end 139.094816 97) (width 0.2) (layer "B.Cu") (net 2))
 (segment (start 141.23153 97) (end 141.39253 96.839) (width 0.2) (layer "B.Cu") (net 2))
 (segment (start 87.5 73) (end 84 73) (width 0.2) (layer "B.Cu") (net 2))
 (segment (start 142.38747 96.839) (end 142.54847 97) (width 0.2) (layer "B.Cu") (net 2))
 (segment (start 168.764 107.085) (end 168.764 106.60824) (width 0.2) (layer "B.Cu") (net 2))
 (segment (start 168.764 106.60824) (end 169.43824 105.934) (width 0.2) (layer "B.Cu") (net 2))
 (segment (start 134.525184 97) (end 135.836184 95.689) (width 0.2) (layer "B.Cu") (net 2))
 (segment (start 171.066 107.085) (end 172.455 107.085) (width 0.2) (layer "B.Cu") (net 2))
 (segment (start 119.58 64.5) (end 124.65 64.5) (width 0.2) (layer "B.Cu") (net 2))
 (segment (start 141.39253 96.839) (end 142.38747 96.839) (width 0.2) (layer "B.Cu") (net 2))
 (segment (start 119.58 64.42) (end 111 73) (width 0.2) (layer "B.Cu") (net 2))
 (segment (start 98.5 70.5) (end 96.5 72.5) (width 0.2) (layer "B.Cu") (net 2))
 (segment (start 111 73) (end 111 95.39) (width 0.2) (layer "B.Cu") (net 2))
 (segment (start 133 95.5) (end 134.5 97) (width 0.2) (layer "B.Cu") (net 2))
 (segment (start 96.5 72.5) (end 88 72.5) (width 0.2) (layer "B.Cu") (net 2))
 (segment (start 134.5 97) (end 134.525184 97) (width 0.2) (layer "B.Cu") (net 2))
 (segment (start 88 72.5) (end 87.5 73) (width 0.2) (layer "B.Cu") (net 2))
 (segment (start 111 95.39) (end 111.11 95.5) (width 0.2) (layer "B.Cu") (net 2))
 (segment (start 171.066 106.60824) (end 171.066 107.085) (width 0.2) (layer "B.Cu") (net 2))
 (segment (start 168.526 106.60824) (end 168.526 107.085) (width 0.2) (layer "B.Cu") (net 2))
 (segment (start 167.85176 105.934) (end 168.526 106.60824) (width 0.2) (layer "B.Cu") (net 2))
 (segment (start 119.58 33.05) (end 119.58 64.42) (width 0.2) (layer "B.Cu") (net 2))
 (segment (start 111.11 95.5) (end 133 95.5) (width 0.2) (layer "B.Cu") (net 2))
 (segment (start 167.375 106.8079) (end 167.375 107.085) (width 0.2) (layer "F.Cu") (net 5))
 (segment (start 118.39 71.5) (end 138.558686 71.5) (width 0.2) (layer "F.Cu") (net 5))
 (segment (start 140.861 78.361) (end 151 88.5) (width 0.2) (layer "F.Cu") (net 5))
 (segment (start 138.558686 71.5) (end 138.059 71.000314) (width 0.2) (layer "F.Cu") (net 5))
 (segment (start 140.861 76.05947) (end 140.861 78.361) (width 0.2) (layer "F.Cu") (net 5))
 (segment (start 138.059 71.000314) (end 138.059 69.839686) (width 0.2) (layer "F.Cu") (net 5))
 (segment (start 151 90.4329) (end 167.375 106.8079) (width 0.2) (layer "F.Cu") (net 5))
 (segment (start 138.879686 69.019) (end 140.040314 69.019) (width 0.2) (layer "F.Cu") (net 5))
 (segment (start 138.059 69.839686) (end 138.879686 69.019) (width 0.2) (layer "F.Cu") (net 5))
 (segment (start 151 88.5) (end 151 90.4329) (width 0.2) (layer "F.Cu") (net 5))
 (segment (start 140.040314 69.019) (end 140.861 69.839686) (width 0.2) (layer "F.Cu") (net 5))
 (segment (start 140.861 73.5) (end 140.799 75.00253) (width 0.2) (layer "F.Cu") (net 5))
 (segment (start 117.35 70.46) (end 118.39 71.5) (width 0.2) (layer "F.Cu") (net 5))
 (segment (start 140.799 75.00253) (end 140.799 75.99747) (width 0.2) (layer "F.Cu") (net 5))
 (segment (start 140.799 75.99747) (end 140.861 76.05947) (width 0.2) (layer "F.Cu") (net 5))
 (segment (start 140.861 69.839686) (end 140.861 73.5) (width 0.2) (layer "F.Cu") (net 5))
 (segment (start 162.484 105.984) (end 162.77176 105.984) (width 0.2) (layer "F.Cu") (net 4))
 (segment (start 139.46 70.42) (end 139.46 82.96) (width 0.2) (layer "F.Cu") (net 4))
 (segment (start 163.446 106.65824) (end 163.446 106.946) (width 0.2) (layer "F.Cu") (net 4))
 (segment (start 163.585 107.085) (end 164.835 107.085) (width 0.2) (layer "F.Cu") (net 4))
 (segment (start 163.446 106.946) (end 163.585 107.085) (width 0.2) (layer "F.Cu") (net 4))
 (segment (start 139.46 82.96) (end 162.484 105.984) (width 0.2) (layer "F.Cu") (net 4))
 (segment (start 162.77176 105.984) (end 163.446 106.65824) (width 0.2) (layer "F.Cu") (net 4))
 (segment (start 161.194 105.984) (end 162.295 107.085) (width 0.2) (layer "F.Cu") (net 3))
 (segment (start 117.46 92.96) (end 130.484 105.984) (width 0.2) (layer "F.Cu") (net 3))
 (segment (start 130.484 105.984) (end 161.194 105.984) (width 0.2) (layer "F.Cu") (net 3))
 (segment (start 168 85.17) (end 164.835 88.335) (width 0.2) (layer "F.Cu") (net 11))
 (segment (start 164.835 88.335) (end 164.835 91.835) (width 0.2) (layer "F.Cu") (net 11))
 (segment (start 127.2 33.05) (end 127.2 43.2) (width 0.2) (layer "F.Cu") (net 11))
 (segment (start 168 84) (end 168 85.17) (width 0.2) (layer "F.Cu") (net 11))
 (segment (start 127.2 43.2) (end 168 84) (width 0.2) (layer "F.Cu") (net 11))
 (segment (start 162.295 81.57855) (end 162.295 91.835) (width 0.2) (layer "F.Cu") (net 10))
 (segment (start 124.66 33.05) (end 124.66 43.94355) (width 0.2) (layer "F.Cu") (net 10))
 (segment (start 124.66 43.94355) (end 162.295 81.57855) (width 0.2) (layer "F.Cu") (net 10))
 (segment (start 122.12 33.05) (end 122.12 47.12) (width 0.2) (layer "F.Cu") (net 9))
 (segment (start 122.12 47.12) (end 161.144 86.144) (width 0.2) (layer "F.Cu") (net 9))
 (segment (start 161.144 86.144) (end 161.144 98.314) (width 0.2) (layer "F.Cu") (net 9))
 (segment (start 161.144 98.314) (end 169.915 107.085) (width 0.2) (layer "F.Cu") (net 9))
 (segment (start 127.656049 31.749) (end 128.301 32.393951) (width 0.2) (layer "F.Cu") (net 6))
 (segment (start 169.915 81.415) (end 169.915 91.835) (width 0.2) (layer "F.Cu") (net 6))
 (segment (start 128.301 32.393951) (end 128.301 39.7339) (width 0.2) (layer "F.Cu") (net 6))
 (segment (start 120.681 34.351) (end 120.681 32.731951) (width 0.2) (layer "F.Cu") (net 6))
 (segment (start 120.5 34.351) (end 120.681 34.351) (width 0.2) (layer "F.Cu") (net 6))
 (segment (start 101.5061 66.099) (end 120.5 47.1051) (width 0.2) (layer "F.Cu") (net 6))
 (segment (start 120.5 47.1051) (end 120.5 34.351) (width 0.2) (layer "F.Cu") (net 6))
 (segment (start 128.301 39.7339) (end 168.401 79.8339) (width 0.2) (layer "F.Cu") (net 6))
 (segment (start 121.663951 31.749) (end 127.656049 31.749) (width 0.2) (layer "F.Cu") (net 6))
 (segment (start 120.681 32.731951) (end 121.663951 31.749) (width 0.2) (layer "F.Cu") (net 6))
 (segment (start 84 70.5) (end 88.401 66.099) (width 0.2) (layer "F.Cu") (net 6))
 (segment (start 168.401 79.8339) (end 168.401 79.901) (width 0.2) (layer "F.Cu") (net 6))
 (segment (start 168.401 79.901) (end 169.915 81.415) (width 0.2) (layer "F.Cu") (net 6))
 (segment (start 88.401 66.099) (end 101.5061 66.099) (width 0.2) (layer "F.Cu") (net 6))
 (segment (start 118.1839 69.059) (end 118.6249 68.618) (width 0.2) (layer "F.Cu") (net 7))
 (segment (start 90.441 69.059) (end 118.1839 69.059) (width 0.2) (layer "F.Cu") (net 7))
 (segment (start 142 69.5) (end 142 70) (width 0.2) (layer "F.Cu") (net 7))
 (segment (start 138.118 68.618) (end 138.236 68.5) (width 0.2) (layer "F.Cu") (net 7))
 (segment (start 142 70) (end 160 88) (width 0.2) (layer "F.Cu") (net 7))
 (segment (start 138.831586 68.5) (end 139.331586 68) (width 0.2) (layer "F.Cu") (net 7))
 (segment (start 84 75.5) (end 90.441 69.059) (width 0.2) (layer "F.Cu") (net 7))
 (segment (start 140.5 68) (end 142 69.5) (width 0.2) (layer "F.Cu") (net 7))
 (segment (start 138.236 68.5) (end 138.831586 68.5) (width 0.2) (layer "F.Cu") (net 7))
 (segment (start 160 88) (end 160 88.5) (width 0.2) (layer "F.Cu") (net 7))
 (segment (start 139.331586 68) (end 140.5 68) (width 0.2) (layer "F.Cu") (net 7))
 (segment (start 118.6249 68.618) (end 138.118 68.618) (width 0.2) (layer "F.Cu") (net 7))
 (segment (start 98.5 75.981314) (end 116.879686 94.361) (width 0.2) (layer "F.Cu") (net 8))
 (segment (start 116.879686 96.67487) (end 117.271 97.066184) (width 0.2) (layer "F.Cu") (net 8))
 (segment (start 128 109.5) (end 157.34 109.5) (width 0.2) (layer "F.Cu") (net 8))
 (segment (start 117.271 97.066184) (end 117.271 98.771) (width 0.2) (layer "F.Cu") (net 8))
 (segment (start 98.5 75.5) (end 98.5 75.981314) (width 0.2) (layer "F.Cu") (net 8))
 (segment (start 117.271 98.771) (end 128 109.5) (width 0.2) (layer "F.Cu") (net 8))
 (segment (start 157.34 109.5) (end 159.755 107.085) (width 0.2) (layer "F.Cu") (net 8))
 (segment (start 116.879686 94.361) (end 116.879686 96.67487) (width 0.2) (layer "F.Cu") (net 8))
 (segment (start 166.25 92.96) (end 167.375 91.835) (width 0.2) (layer "B.Cu") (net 1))
 (segment (start 139.35 92.96) (end 139.46 92.96) (width 0.2) (layer "B.Cu") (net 1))
 (segment (start 139.5 93) (end 139 93) (width 0.2) (layer "B.Cu") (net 1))
 (segment (start 139.46 92.96) (end 139.5 93) (width 0.2) (layer "B.Cu") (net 1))
 (segment (start 139.35 92.96) (end 166.25 92.96) (width 0.2) (layer "B.Cu") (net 1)))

